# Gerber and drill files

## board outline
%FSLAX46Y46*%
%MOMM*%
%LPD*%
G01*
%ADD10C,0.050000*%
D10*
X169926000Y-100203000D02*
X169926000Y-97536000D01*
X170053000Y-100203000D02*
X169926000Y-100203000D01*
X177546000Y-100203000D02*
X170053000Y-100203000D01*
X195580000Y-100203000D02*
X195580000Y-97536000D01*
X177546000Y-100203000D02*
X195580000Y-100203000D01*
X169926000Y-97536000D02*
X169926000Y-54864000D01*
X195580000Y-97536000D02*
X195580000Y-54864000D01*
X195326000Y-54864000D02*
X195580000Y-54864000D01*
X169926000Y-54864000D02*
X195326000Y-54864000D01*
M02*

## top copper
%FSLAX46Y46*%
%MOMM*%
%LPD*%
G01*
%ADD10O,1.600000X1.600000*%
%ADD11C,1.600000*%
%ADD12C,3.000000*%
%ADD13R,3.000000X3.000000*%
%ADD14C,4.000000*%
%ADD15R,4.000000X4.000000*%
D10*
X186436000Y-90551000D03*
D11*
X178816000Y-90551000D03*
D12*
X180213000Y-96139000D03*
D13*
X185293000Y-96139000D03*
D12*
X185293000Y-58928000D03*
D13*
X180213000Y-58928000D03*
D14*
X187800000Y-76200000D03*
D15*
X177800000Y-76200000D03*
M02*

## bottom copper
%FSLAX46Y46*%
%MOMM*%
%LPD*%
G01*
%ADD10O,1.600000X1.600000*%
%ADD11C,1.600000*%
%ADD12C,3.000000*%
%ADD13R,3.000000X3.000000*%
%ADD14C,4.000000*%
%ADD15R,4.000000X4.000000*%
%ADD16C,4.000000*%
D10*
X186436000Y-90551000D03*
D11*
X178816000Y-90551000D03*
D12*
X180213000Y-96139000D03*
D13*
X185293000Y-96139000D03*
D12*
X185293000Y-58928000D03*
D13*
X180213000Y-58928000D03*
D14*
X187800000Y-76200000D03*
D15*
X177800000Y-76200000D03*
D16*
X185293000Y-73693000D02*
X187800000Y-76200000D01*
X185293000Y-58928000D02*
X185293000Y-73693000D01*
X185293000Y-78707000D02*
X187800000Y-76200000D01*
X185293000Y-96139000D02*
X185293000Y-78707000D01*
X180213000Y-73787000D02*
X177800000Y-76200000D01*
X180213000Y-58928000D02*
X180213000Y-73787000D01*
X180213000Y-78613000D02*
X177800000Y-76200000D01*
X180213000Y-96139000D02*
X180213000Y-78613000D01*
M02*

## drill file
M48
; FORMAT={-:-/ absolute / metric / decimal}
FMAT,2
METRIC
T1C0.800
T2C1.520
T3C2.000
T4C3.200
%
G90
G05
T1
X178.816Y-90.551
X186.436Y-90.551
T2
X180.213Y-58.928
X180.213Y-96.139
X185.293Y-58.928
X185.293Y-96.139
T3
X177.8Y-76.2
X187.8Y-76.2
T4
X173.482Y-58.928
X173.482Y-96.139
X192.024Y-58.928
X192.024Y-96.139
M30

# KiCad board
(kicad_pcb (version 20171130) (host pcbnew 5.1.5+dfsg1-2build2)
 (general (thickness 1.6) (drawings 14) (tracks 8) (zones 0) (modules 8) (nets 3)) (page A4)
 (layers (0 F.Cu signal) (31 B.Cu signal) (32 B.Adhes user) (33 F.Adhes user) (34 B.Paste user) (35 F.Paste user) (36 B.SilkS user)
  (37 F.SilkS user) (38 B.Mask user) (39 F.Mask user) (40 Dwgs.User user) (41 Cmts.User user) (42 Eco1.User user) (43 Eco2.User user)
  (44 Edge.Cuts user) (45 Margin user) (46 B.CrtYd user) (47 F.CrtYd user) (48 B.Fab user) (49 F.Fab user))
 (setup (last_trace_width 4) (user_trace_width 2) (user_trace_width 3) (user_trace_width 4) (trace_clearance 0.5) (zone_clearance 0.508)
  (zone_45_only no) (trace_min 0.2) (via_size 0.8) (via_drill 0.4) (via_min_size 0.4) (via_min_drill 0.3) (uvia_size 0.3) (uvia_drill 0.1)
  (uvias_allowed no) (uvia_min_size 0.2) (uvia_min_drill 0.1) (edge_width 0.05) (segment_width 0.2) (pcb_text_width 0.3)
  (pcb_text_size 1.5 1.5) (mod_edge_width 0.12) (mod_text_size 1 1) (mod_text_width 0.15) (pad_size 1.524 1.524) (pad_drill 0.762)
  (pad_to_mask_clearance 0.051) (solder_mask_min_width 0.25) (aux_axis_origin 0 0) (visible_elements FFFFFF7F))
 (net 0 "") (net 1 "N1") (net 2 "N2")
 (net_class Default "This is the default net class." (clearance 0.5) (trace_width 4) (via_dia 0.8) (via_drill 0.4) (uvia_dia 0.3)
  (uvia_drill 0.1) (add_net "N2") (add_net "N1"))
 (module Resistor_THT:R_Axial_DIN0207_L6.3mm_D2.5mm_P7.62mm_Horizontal (layer F.Cu) (at 178.816 90.551)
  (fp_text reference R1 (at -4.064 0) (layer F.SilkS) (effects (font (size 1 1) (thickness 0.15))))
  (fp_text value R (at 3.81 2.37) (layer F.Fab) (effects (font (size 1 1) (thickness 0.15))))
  (pad 2 thru_hole oval (at 7.62 0) (size 1.6 1.6) (drill 0.8) (layers *.Cu *.Mask) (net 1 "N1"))
  (pad 1 thru_hole circle (at 0 0) (size 1.6 1.6) (drill 0.8) (layers *.Cu *.Mask) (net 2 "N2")))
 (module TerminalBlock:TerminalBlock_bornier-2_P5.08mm (layer F.Cu) (at 185.293 96.139 180)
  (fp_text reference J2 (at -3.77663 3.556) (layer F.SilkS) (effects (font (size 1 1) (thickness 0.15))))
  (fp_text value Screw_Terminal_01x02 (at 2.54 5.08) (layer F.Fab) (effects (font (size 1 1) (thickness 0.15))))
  (pad 2 thru_hole circle (at 5.08 0 180) (size 3 3) (drill 1.52) (layers *.Cu *.Mask) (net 2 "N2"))
  (pad 1 thru_hole rect (at 0 0 180) (size 3 3) (drill 1.52) (layers *.Cu *.Mask) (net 1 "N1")))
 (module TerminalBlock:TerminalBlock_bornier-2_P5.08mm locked (layer F.Cu) (at 180.213 58.928)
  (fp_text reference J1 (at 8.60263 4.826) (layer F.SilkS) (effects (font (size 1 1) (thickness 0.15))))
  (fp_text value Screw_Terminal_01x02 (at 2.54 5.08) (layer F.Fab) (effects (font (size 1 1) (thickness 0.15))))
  (pad 2 thru_hole circle (at 5.08 0) (size 3 3) (drill 1.52) (layers *.Cu *.Mask) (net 1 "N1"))
  (pad 1 thru_hole rect (at 0 0) (size 3 3) (drill 1.52) (layers *.Cu *.Mask) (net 2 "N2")))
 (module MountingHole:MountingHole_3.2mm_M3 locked (layer F.Cu) (at 192.024 96.139)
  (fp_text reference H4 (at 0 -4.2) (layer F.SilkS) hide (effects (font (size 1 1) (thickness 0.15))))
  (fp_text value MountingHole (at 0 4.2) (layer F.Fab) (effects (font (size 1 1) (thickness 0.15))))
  (pad 1 np_thru_hole circle (at 0 0) (size 3.2 3.2) (drill 3.2) (layers *.Cu *.Mask)))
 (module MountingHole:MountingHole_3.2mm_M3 (layer F.Cu) (at 173.482 96.139)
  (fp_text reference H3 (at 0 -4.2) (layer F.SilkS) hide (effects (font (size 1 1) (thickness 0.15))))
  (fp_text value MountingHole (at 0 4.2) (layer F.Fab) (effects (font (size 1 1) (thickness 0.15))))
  (pad 1 np_thru_hole circle (at 0 0) (size 3.2 3.2) (drill 3.2) (layers *.Cu *.Mask)))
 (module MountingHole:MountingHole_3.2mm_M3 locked (layer F.Cu) (at 192.024 58.928)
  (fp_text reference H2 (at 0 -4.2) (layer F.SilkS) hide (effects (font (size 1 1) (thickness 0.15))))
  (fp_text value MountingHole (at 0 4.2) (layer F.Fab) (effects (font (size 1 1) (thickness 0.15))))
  (pad 1 np_thru_hole circle (at 0 0) (size 3.2 3.2) (drill 3.2) (layers *.Cu *.Mask)))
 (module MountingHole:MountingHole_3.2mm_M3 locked (layer F.Cu) (at 173.482 58.928)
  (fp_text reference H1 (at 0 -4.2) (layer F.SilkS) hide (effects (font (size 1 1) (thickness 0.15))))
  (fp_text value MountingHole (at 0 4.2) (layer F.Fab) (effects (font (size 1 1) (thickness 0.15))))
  (pad 1 np_thru_hole circle (at 0 0) (size 3.2 3.2) (drill 3.2) (layers *.Cu *.Mask)))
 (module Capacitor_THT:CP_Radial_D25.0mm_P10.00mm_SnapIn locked (layer F.Cu) (at 177.8 76.2)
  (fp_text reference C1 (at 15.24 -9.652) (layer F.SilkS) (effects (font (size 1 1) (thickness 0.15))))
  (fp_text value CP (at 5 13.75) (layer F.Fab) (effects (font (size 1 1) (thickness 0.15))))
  (pad 2 thru_hole circle (at 10 0) (size 4 4) (drill 2) (layers *.Cu *.Mask) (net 1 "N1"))
  (pad 1 thru_hole rect (at 0 0) (size 4 4) (drill 2) (layers *.Cu *.Mask) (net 2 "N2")))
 (gr_line (start 169.926 100.203) (end 169.926 97.536) (layer Edge.Cuts) (width 0.05))
 (gr_line (start 170.053 100.203) (end 169.926 100.203) (layer Edge.Cuts) (width 0.05))
 (gr_line (start 177.546 100.203) (end 170.053 100.203) (layer Edge.Cuts) (width 0.05))
 (gr_line (start 195.58 100.203) (end 195.58 97.536) (layer Edge.Cuts) (width 0.05))
 (gr_line (start 177.546 100.203) (end 195.58 100.203) (layer Edge.Cuts) (width 0.05))
 (gr_line (start 169.926 97.536) (end 169.926 54.864) (layer Edge.Cuts) (width 0.05))
 (gr_line (start 195.58 97.536) (end 195.58 54.864) (layer Edge.Cuts) (width 0.05))
 (gr_line (start 195.326 54.864) (end 195.58 54.864) (layer Edge.Cuts) (width 0.05))
 (gr_line (start 169.926 54.864) (end 195.326 54.864) (layer Edge.Cuts) (width 0.05))
 (segment (start 185.293 73.693) (end 187.8 76.2) (width 4) (layer B.Cu) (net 1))
 (segment (start 185.293 58.928) (end 185.293 73.693) (width 4) (layer B.Cu) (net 1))
 (segment (start 185.293 78.707) (end 187.8 76.2) (width 4) (layer B.Cu) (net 1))
 (segment (start 185.293 96.139) (end 185.293 78.707) (width 4) (layer B.Cu) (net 1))
 (segment (start 180.213 73.787) (end 177.8 76.2) (width 4) (layer B.Cu) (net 2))
 (segment (start 180.213 58.928) (end 180.213 73.787) (width 4) (layer B.Cu) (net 2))
 (segment (start 180.213 78.613) (end 177.8 76.2) (width 4) (layer B.Cu) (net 2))
 (segment (start 180.213 96.139) (end 180.213 78.613) (width 4) (layer B.Cu) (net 2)))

